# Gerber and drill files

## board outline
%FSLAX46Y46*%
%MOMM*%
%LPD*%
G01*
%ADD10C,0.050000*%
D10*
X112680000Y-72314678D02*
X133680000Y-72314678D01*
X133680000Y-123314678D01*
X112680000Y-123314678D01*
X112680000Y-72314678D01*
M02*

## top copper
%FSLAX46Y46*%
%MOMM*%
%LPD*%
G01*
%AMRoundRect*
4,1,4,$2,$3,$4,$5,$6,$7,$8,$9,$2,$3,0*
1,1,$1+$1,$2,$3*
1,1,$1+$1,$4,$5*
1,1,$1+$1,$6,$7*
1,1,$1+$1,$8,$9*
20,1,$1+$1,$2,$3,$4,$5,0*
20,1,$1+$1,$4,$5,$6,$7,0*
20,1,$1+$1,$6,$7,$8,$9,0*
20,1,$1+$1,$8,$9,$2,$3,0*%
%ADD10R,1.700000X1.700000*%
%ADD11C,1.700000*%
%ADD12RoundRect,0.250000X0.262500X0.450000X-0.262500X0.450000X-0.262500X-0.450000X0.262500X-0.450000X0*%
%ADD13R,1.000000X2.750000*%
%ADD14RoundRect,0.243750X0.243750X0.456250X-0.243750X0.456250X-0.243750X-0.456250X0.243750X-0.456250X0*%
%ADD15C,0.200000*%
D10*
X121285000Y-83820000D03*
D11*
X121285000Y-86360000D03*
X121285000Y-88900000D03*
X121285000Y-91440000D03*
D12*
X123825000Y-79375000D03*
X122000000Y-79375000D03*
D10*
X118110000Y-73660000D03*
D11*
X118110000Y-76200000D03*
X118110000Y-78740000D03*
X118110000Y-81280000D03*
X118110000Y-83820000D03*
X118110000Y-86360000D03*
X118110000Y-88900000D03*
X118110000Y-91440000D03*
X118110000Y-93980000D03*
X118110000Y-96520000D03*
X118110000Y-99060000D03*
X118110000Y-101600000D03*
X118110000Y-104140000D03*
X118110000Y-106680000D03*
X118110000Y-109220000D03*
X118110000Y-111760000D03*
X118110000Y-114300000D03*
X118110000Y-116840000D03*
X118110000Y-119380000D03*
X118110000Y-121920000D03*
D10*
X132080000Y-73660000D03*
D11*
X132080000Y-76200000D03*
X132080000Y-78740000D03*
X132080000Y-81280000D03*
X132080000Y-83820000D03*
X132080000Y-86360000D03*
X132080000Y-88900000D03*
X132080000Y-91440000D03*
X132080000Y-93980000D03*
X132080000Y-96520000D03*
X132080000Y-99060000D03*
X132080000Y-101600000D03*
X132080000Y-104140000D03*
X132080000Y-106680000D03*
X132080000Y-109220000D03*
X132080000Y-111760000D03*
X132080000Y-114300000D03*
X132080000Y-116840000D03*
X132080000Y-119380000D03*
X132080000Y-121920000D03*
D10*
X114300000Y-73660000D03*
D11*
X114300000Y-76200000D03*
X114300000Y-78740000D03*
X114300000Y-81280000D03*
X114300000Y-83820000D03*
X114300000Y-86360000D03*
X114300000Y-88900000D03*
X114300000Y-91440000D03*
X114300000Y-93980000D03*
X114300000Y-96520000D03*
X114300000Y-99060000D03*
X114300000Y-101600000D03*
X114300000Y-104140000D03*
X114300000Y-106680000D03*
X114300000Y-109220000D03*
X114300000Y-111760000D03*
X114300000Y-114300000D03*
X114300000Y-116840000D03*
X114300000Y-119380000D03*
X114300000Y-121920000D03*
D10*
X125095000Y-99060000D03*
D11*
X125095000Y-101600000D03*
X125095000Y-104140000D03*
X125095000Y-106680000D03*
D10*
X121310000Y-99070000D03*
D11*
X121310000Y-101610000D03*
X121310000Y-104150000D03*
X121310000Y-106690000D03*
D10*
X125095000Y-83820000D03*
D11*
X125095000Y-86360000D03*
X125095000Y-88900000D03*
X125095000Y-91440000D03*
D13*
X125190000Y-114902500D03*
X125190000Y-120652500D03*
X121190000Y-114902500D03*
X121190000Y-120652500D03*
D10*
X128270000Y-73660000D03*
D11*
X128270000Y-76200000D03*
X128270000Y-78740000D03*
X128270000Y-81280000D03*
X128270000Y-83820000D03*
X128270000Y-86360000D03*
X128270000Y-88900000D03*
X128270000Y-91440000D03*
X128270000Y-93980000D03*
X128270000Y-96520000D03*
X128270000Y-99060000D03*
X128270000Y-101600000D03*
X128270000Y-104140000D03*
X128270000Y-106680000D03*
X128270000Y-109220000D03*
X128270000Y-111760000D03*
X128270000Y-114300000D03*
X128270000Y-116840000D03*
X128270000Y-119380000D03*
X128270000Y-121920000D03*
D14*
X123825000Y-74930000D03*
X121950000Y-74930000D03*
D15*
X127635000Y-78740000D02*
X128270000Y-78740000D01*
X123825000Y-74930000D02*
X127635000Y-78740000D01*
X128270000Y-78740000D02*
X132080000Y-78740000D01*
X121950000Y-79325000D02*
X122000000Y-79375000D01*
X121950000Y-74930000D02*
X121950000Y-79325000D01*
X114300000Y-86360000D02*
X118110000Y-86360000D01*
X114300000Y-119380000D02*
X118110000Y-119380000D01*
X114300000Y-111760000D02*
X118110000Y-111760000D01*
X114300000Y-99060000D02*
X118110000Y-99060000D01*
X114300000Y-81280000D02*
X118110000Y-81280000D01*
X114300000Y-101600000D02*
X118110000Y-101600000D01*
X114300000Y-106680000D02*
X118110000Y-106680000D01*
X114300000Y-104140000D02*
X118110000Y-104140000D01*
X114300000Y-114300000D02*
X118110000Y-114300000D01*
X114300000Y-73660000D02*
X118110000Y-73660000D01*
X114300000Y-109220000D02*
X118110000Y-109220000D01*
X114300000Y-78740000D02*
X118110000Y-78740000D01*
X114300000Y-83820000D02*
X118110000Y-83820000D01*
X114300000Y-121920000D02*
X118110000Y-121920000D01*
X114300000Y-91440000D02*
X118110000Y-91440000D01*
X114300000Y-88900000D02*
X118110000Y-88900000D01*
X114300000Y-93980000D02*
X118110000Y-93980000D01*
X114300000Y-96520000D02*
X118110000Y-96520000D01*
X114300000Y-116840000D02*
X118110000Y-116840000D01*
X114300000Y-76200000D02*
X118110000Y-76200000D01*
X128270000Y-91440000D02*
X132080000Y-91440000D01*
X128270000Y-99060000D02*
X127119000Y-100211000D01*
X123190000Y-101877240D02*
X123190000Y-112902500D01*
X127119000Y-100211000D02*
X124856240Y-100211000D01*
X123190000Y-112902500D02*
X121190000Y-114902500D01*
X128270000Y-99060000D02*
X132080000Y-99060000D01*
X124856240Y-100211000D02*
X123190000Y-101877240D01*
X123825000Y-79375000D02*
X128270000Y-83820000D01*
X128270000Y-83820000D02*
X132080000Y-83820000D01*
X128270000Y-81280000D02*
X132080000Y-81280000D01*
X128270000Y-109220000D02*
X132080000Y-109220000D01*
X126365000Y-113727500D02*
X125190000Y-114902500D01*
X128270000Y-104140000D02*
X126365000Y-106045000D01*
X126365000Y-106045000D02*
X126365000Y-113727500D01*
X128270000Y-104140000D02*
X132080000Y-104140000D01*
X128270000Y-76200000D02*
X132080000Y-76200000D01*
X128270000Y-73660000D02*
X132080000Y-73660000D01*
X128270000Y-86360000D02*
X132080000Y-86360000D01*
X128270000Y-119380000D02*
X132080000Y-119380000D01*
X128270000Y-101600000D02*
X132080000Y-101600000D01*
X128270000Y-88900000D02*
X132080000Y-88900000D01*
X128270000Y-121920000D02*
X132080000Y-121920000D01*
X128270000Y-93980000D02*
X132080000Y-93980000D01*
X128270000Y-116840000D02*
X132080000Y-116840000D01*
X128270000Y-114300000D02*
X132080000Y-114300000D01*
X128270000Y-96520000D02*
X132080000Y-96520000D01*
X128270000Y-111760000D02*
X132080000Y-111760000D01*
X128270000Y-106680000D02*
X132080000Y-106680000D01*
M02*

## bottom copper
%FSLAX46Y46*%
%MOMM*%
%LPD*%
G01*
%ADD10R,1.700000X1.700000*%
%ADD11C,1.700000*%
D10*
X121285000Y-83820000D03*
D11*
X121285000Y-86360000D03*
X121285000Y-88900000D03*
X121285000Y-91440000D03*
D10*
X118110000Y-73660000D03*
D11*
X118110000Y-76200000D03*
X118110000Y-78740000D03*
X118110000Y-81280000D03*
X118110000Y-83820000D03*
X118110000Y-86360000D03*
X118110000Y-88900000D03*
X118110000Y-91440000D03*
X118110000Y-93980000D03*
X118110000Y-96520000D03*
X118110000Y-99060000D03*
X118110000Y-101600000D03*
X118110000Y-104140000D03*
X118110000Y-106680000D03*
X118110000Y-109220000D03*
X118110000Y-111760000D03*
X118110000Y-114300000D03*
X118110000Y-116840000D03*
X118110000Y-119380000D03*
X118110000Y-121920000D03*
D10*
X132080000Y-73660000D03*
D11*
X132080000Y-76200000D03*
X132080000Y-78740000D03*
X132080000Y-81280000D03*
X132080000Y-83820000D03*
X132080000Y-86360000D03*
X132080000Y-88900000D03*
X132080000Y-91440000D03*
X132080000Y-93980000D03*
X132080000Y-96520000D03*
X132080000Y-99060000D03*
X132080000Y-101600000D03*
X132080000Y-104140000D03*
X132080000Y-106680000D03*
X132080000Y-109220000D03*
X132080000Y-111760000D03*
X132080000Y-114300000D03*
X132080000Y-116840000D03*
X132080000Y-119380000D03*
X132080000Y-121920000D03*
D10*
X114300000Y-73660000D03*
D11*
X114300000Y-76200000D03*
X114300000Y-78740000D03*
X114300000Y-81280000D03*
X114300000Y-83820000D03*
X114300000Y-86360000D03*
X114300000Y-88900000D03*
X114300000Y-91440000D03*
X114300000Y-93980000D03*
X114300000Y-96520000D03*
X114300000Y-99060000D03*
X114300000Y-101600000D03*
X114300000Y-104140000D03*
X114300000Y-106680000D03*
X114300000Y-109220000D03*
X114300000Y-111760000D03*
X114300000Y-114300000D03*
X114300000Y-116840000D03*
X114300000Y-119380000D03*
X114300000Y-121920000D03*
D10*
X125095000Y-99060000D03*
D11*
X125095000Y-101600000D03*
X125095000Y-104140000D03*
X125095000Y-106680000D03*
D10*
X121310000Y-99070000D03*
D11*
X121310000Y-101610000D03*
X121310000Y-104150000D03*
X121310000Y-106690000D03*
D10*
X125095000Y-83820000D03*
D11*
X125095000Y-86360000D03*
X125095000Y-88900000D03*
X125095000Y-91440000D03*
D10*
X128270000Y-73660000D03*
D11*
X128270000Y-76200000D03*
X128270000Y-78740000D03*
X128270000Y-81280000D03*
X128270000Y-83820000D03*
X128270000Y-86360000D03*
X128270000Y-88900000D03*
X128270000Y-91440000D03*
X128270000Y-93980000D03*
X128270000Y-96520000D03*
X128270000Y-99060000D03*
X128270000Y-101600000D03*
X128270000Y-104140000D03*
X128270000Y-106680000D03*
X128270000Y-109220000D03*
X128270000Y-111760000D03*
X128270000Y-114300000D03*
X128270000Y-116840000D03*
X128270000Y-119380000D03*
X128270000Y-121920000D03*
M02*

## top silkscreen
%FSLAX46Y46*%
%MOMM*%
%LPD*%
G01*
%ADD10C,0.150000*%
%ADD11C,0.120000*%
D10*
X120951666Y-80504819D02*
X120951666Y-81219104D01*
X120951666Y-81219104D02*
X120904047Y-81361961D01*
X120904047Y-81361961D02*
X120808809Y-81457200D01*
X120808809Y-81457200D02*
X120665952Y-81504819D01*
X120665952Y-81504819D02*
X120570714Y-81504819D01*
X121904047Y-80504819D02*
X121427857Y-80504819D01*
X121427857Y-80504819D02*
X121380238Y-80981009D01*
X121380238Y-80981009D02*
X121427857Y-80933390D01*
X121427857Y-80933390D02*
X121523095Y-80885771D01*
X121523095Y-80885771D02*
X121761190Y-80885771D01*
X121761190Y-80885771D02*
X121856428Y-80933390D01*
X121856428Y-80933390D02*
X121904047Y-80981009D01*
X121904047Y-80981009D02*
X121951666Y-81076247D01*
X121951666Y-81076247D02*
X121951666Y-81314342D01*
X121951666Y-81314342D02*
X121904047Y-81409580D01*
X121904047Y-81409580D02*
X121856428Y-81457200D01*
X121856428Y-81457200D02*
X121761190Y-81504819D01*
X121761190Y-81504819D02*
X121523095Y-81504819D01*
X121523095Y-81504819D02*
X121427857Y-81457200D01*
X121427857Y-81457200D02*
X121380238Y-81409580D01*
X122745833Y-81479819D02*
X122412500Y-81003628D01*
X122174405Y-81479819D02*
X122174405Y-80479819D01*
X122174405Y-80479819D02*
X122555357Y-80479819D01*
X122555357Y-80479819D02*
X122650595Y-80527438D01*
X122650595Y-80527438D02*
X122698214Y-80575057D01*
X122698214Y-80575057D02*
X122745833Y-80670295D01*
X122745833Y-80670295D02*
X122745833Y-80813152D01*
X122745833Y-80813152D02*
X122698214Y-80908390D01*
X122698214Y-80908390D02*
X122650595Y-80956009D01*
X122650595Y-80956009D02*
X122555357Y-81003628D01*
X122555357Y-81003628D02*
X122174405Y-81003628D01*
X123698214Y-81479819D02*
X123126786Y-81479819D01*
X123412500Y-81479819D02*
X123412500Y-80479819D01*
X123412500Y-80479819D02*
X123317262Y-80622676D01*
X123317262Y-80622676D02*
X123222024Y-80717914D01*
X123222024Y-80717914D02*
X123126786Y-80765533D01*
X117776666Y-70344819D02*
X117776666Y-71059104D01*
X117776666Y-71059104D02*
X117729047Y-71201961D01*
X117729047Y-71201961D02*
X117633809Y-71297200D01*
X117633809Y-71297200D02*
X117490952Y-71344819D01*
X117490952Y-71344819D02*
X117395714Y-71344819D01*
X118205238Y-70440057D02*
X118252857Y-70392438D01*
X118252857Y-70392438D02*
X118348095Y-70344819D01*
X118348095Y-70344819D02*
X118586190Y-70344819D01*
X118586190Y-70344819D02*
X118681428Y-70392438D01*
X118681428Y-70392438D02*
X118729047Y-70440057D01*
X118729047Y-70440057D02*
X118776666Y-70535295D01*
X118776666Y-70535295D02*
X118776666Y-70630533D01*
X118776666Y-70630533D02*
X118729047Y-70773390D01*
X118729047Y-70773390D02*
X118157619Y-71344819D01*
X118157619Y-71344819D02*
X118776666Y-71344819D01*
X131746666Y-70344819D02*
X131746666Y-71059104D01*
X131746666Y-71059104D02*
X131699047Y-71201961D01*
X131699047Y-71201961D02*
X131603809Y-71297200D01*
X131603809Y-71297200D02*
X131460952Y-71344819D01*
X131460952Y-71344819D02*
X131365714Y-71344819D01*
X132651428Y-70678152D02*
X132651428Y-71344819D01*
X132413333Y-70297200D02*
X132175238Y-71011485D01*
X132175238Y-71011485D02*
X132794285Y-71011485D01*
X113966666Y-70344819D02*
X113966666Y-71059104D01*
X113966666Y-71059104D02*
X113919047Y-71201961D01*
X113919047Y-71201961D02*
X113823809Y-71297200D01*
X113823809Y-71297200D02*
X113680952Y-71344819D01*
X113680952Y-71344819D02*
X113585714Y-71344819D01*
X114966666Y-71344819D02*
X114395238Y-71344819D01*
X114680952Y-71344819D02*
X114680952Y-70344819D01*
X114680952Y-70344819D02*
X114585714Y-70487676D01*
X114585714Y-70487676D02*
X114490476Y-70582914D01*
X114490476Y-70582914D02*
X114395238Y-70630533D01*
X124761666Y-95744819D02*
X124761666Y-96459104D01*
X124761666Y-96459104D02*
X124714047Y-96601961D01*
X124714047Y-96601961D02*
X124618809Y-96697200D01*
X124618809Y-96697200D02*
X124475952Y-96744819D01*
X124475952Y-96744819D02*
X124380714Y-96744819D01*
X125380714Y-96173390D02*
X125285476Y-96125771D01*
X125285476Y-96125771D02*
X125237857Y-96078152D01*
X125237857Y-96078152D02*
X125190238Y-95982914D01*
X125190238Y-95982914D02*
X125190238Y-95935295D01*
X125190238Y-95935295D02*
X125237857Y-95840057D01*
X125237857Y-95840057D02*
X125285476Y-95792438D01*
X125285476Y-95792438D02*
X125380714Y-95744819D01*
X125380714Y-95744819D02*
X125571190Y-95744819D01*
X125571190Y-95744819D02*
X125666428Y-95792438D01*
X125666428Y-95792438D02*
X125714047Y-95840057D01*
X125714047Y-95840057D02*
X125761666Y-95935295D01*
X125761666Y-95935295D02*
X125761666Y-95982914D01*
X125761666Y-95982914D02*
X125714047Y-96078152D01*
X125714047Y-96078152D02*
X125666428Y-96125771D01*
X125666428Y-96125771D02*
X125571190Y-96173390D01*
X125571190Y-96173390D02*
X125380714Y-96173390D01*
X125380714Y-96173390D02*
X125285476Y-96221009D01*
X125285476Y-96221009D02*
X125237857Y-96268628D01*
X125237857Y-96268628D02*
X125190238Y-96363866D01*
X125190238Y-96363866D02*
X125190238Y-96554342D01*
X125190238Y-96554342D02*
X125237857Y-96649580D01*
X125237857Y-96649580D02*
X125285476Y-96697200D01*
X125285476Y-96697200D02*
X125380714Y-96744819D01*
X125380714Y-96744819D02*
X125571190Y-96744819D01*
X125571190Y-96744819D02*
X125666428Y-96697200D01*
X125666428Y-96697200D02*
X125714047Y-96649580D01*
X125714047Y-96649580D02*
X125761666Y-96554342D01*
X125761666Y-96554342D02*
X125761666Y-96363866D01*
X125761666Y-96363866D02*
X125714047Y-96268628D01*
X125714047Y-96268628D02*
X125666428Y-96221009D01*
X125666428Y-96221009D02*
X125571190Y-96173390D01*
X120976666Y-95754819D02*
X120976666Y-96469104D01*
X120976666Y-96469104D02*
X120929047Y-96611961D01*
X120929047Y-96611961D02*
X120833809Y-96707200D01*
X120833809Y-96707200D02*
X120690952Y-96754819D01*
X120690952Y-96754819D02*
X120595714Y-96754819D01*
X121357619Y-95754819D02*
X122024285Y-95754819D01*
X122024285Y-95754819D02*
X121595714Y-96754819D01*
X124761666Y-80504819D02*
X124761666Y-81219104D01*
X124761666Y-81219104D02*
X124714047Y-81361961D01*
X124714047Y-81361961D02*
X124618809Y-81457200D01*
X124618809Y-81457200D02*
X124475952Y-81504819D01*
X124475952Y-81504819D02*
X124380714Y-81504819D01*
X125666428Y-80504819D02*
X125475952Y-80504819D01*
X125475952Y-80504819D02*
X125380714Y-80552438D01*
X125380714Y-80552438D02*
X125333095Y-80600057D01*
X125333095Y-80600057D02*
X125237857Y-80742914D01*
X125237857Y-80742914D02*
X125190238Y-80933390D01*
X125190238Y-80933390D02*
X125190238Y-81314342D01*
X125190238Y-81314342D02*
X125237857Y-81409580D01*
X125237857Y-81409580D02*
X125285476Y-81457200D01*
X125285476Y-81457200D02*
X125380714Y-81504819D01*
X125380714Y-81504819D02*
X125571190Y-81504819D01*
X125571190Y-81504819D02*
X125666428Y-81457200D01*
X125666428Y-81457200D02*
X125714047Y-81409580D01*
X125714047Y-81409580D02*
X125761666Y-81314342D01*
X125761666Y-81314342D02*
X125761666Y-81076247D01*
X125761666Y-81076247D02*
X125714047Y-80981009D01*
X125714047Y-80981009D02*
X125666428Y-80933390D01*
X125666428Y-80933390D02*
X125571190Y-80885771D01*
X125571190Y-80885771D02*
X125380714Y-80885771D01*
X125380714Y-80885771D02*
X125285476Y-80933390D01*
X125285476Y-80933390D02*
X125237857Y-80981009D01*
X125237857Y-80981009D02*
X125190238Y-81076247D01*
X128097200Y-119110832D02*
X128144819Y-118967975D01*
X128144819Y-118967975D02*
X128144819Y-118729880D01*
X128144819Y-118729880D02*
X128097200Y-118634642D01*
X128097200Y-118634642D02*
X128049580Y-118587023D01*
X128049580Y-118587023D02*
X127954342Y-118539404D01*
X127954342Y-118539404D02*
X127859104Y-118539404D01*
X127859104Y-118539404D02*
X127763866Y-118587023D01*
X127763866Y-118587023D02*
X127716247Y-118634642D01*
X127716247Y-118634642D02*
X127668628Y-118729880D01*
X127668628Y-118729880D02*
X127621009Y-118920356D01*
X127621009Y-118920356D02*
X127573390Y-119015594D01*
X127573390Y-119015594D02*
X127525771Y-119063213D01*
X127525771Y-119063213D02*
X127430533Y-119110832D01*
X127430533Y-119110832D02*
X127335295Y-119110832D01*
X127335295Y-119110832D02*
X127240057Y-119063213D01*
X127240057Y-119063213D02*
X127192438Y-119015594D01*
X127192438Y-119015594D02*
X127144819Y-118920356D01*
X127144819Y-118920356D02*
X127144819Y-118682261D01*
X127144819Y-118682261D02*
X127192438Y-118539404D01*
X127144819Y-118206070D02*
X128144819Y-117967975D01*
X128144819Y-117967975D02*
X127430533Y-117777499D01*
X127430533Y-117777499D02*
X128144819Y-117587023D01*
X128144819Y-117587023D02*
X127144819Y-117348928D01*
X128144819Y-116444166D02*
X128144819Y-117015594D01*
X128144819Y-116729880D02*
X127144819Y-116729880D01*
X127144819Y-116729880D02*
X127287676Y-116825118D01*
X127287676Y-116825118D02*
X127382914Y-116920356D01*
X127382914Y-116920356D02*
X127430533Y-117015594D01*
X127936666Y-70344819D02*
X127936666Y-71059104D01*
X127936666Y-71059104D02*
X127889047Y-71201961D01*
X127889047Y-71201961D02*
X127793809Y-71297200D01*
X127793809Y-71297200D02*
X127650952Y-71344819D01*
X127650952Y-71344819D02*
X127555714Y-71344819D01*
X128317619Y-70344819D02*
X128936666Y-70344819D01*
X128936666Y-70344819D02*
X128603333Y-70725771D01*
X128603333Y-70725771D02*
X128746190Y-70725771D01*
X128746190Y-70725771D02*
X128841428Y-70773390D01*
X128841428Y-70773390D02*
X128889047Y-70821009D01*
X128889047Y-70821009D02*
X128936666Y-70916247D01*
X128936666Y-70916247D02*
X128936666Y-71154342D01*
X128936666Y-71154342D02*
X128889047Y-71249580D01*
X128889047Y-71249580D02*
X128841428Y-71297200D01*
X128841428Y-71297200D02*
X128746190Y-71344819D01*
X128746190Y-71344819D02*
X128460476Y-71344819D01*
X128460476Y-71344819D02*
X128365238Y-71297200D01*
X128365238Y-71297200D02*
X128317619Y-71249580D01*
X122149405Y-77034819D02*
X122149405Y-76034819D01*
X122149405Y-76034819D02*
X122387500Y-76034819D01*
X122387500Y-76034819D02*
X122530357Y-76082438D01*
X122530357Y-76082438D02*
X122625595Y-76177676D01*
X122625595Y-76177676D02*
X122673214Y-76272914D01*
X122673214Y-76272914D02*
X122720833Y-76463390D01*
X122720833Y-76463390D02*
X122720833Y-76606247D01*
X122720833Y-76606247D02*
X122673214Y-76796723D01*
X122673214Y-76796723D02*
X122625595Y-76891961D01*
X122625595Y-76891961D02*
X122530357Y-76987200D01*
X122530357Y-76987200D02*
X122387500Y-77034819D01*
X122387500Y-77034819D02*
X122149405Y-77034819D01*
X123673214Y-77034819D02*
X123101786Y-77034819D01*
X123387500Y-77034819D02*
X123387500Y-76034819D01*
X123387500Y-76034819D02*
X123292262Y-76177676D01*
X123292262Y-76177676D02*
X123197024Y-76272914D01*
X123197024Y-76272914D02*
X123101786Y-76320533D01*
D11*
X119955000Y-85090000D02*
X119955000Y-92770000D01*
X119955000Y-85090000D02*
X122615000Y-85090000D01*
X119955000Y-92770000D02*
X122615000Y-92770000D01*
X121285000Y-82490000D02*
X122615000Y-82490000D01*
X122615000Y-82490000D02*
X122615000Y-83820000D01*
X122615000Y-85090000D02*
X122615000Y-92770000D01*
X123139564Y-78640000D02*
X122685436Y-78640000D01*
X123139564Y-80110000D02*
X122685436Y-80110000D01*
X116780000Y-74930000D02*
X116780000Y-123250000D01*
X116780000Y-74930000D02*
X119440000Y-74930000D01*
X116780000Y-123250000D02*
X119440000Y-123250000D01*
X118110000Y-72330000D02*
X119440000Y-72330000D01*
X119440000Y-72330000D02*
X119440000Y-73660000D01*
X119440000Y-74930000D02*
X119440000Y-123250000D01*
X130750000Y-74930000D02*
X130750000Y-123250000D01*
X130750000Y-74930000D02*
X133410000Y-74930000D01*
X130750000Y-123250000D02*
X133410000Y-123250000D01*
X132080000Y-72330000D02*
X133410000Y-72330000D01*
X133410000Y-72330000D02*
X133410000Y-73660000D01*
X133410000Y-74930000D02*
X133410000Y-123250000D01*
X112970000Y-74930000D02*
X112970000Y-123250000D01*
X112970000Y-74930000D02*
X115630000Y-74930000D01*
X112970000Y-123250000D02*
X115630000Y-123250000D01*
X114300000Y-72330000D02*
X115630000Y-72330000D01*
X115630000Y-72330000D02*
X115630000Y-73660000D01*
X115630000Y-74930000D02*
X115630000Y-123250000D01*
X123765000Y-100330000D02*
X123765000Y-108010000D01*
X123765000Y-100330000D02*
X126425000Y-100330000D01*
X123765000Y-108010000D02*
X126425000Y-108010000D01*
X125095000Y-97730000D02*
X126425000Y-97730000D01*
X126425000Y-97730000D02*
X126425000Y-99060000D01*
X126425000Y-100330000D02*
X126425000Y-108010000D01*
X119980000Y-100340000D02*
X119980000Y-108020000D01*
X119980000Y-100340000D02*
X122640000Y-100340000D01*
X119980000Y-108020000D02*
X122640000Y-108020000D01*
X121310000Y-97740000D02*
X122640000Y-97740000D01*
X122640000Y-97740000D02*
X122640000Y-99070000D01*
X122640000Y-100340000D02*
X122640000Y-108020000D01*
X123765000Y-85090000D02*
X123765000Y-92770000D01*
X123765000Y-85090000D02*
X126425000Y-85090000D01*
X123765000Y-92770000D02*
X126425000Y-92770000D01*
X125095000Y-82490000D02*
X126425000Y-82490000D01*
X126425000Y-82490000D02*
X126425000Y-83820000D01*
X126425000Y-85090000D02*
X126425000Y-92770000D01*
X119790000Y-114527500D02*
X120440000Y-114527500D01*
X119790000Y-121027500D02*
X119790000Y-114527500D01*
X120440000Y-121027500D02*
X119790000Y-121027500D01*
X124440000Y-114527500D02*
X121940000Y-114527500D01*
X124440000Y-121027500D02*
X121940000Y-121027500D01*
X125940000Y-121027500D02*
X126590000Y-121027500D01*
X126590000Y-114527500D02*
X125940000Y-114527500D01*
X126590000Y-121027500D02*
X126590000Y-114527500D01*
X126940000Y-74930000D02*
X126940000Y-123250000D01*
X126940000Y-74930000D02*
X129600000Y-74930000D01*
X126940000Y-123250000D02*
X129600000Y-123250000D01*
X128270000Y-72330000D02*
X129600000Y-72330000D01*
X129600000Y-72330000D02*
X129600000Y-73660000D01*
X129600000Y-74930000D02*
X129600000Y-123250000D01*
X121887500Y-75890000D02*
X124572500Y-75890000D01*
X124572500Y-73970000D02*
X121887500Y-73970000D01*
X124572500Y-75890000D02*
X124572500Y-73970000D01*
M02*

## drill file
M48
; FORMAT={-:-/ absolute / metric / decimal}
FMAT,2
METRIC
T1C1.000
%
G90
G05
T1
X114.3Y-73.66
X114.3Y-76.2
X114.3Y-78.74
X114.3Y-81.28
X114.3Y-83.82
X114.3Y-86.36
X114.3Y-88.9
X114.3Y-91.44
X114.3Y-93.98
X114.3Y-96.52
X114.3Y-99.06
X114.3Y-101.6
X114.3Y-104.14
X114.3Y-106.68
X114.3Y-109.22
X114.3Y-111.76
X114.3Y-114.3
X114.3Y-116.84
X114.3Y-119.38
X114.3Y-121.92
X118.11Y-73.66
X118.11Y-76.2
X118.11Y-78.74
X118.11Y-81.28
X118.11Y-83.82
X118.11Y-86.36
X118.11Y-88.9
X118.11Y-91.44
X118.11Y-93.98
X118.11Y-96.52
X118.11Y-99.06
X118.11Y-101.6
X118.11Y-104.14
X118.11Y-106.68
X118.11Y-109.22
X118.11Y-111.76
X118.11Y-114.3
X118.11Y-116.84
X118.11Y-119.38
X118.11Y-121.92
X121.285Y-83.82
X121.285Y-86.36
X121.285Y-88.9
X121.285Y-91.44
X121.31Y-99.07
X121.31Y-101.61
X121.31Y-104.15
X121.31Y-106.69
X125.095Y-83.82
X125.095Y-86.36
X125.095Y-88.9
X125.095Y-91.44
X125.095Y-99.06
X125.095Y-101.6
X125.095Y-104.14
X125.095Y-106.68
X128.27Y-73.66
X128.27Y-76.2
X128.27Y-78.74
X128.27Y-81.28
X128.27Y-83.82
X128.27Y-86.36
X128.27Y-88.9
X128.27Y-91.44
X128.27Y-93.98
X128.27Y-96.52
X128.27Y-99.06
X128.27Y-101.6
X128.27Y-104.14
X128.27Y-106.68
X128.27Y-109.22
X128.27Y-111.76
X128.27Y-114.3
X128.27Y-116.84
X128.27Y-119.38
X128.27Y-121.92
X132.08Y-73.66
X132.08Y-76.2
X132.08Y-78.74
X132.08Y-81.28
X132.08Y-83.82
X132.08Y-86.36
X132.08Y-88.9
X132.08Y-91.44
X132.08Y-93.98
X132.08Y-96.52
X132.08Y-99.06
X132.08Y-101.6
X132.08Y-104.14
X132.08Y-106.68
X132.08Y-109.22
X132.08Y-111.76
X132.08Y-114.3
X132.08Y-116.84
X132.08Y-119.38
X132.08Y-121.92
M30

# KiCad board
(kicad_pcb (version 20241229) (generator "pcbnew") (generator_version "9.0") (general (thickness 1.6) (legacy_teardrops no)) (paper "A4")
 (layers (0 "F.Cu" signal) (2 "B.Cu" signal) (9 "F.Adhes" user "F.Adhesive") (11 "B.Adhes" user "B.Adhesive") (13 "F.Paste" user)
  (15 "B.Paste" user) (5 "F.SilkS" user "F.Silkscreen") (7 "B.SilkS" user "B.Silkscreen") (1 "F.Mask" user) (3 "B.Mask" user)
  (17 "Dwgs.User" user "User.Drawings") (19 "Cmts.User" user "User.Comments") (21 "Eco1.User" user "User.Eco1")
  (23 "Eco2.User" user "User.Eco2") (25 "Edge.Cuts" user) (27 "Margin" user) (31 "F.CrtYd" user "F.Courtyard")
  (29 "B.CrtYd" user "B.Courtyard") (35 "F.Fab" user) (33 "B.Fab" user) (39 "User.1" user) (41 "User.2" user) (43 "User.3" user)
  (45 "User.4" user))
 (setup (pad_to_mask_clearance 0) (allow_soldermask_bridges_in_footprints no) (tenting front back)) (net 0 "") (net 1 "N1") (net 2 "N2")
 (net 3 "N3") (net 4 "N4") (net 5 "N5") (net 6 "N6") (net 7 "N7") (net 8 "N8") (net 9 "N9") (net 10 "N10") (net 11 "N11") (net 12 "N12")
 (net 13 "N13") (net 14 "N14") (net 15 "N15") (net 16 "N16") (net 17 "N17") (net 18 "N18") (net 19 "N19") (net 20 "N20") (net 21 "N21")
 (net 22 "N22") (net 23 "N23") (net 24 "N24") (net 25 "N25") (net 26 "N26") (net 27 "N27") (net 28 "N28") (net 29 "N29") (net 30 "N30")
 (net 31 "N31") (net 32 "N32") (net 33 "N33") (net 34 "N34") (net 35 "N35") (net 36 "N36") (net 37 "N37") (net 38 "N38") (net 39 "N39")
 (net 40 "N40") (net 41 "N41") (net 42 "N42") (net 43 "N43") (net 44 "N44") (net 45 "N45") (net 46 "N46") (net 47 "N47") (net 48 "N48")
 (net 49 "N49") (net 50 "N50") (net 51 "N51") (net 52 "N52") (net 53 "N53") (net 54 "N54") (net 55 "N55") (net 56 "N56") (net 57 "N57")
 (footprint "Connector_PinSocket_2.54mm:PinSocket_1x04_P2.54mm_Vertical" (layer "F.Cu") (at 121.285 83.82)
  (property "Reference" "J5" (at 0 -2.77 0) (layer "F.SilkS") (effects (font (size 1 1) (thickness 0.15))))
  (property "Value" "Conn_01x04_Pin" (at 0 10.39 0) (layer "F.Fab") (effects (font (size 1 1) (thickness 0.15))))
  (fp_line (start -1.33 1.27) (end -1.33 8.95) (stroke (width 0.12) (type solid)) (layer "F.SilkS"))
  (fp_line (start -1.33 1.27) (end 1.33 1.27) (stroke (width 0.12) (type solid)) (layer "F.SilkS"))
  (fp_line (start -1.33 8.95) (end 1.33 8.95) (stroke (width 0.12) (type solid)) (layer "F.SilkS"))
  (fp_line (start 0 -1.33) (end 1.33 -1.33) (stroke (width 0.12) (type solid)) (layer "F.SilkS"))
  (fp_line (start 1.33 -1.33) (end 1.33 0) (stroke (width 0.12) (type solid)) (layer "F.SilkS"))
  (fp_line (start 1.33 1.27) (end 1.33 8.95) (stroke (width 0.12) (type solid)) (layer "F.SilkS"))
  (pad "1" thru_hole rect (at 0 0) (size 1.7 1.7) (drill 1) (layers "*.Cu" "*.Mask") (remove_unused_layers no) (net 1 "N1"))
  (pad "2" thru_hole circle (at 0 2.54) (size 1.7 1.7) (drill 1) (layers "*.Cu" "*.Mask") (remove_unused_layers no) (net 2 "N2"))
  (pad "3" thru_hole circle (at 0 5.08) (size 1.7 1.7) (drill 1) (layers "*.Cu" "*.Mask") (remove_unused_layers no) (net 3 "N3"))
  (pad "4" thru_hole circle (at 0 7.62) (size 1.7 1.7) (drill 1) (layers "*.Cu" "*.Mask") (remove_unused_layers no) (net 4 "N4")))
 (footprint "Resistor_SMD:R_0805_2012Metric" (layer "F.Cu") (at 122.9125 79.375 180)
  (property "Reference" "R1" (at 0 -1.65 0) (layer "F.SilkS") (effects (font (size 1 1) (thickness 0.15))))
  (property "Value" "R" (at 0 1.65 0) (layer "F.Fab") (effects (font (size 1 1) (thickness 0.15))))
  (fp_line (start -0.227064 0.735) (end 0.227064 0.735) (stroke (width 0.12) (type solid)) (layer "F.SilkS"))
  (fp_line (start -0.227064 -0.735) (end 0.227064 -0.735) (stroke (width 0.12) (type solid)) (layer "F.SilkS"))
  (pad "1" smd roundrect (at -0.9125 0 180) (size 1.025 1.4) (layers "F.Cu" "F.Mask" "F.Paste") (roundrect_rratio 0.243902) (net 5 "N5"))
  (pad "2" smd roundrect (at 0.9125 0 180) (size 1.025 1.4) (layers "F.Cu" "F.Mask" "F.Paste") (roundrect_rratio 0.243902) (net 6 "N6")))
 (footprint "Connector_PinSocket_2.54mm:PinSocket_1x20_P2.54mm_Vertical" (layer "F.Cu") (at 118.11 73.66)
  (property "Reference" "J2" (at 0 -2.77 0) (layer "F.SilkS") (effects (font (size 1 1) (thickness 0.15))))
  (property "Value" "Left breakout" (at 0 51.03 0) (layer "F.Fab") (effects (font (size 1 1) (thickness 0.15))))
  (fp_line (start -1.33 1.27) (end -1.33 49.59) (stroke (width 0.12) (type solid)) (layer "F.SilkS"))
  (fp_line (start -1.33 1.27) (end 1.33 1.27) (stroke (width 0.12) (type solid)) (layer "F.SilkS"))
  (fp_line (start -1.33 49.59) (end 1.33 49.59) (stroke (width 0.12) (type solid)) (layer "F.SilkS"))
  (fp_line (start 0 -1.33) (end 1.33 -1.33) (stroke (width 0.12) (type solid)) (layer "F.SilkS"))
  (fp_line (start 1.33 -1.33) (end 1.33 0) (stroke (width 0.12) (type solid)) (layer "F.SilkS"))
  (fp_line (start 1.33 1.27) (end 1.33 49.59) (stroke (width 0.12) (type solid)) (layer "F.SilkS"))
  (pad "1" thru_hole rect (at 0 0) (size 1.7 1.7) (drill 1) (layers "*.Cu" "*.Mask") (remove_unused_layers no) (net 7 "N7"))
  (pad "2" thru_hole circle (at 0 2.54) (size 1.7 1.7) (drill 1) (layers "*.Cu" "*.Mask") (remove_unused_layers no) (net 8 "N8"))
  (pad "3" thru_hole circle (at 0 5.08) (size 1.7 1.7) (drill 1) (layers "*.Cu" "*.Mask") (remove_unused_layers no) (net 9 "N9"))
  (pad "4" thru_hole circle (at 0 7.62) (size 1.7 1.7) (drill 1) (layers "*.Cu" "*.Mask") (remove_unused_layers no) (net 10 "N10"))
  (pad "5" thru_hole circle (at 0 10.16) (size 1.7 1.7) (drill 1) (layers "*.Cu" "*.Mask") (remove_unused_layers no) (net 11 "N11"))
  (pad "6" thru_hole circle (at 0 12.7) (size 1.7 1.7) (drill 1) (layers "*.Cu" "*.Mask") (remove_unused_layers no) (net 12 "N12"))
  (pad "7" thru_hole circle (at 0 15.24) (size 1.7 1.7) (drill 1) (layers "*.Cu" "*.Mask") (remove_unused_layers no) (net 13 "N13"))
  (pad "8" thru_hole circle (at 0 17.78) (size 1.7 1.7) (drill 1) (layers "*.Cu" "*.Mask") (remove_unused_layers no) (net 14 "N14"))
  (pad "9" thru_hole circle (at 0 20.32) (size 1.7 1.7) (drill 1) (layers "*.Cu" "*.Mask") (remove_unused_layers no) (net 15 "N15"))
  (pad "10" thru_hole circle (at 0 22.86) (size 1.7 1.7) (drill 1) (layers "*.Cu" "*.Mask") (remove_unused_layers no) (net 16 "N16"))
  (pad "11" thru_hole circle (at 0 25.4) (size 1.7 1.7) (drill 1) (layers "*.Cu" "*.Mask") (remove_unused_layers no) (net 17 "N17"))
  (pad "12" thru_hole circle (at 0 27.94) (size 1.7 1.7) (drill 1) (layers "*.Cu" "*.Mask") (remove_unused_layers no) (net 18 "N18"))
  (pad "13" thru_hole circle (at 0 30.48) (size 1.7 1.7) (drill 1) (layers "*.Cu" "*.Mask") (remove_unused_layers no) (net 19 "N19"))
  (pad "14" thru_hole circle (at 0 33.02) (size 1.7 1.7) (drill 1) (layers "*.Cu" "*.Mask") (remove_unused_layers no) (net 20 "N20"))
  (pad "15" thru_hole circle (at 0 35.56) (size 1.7 1.7) (drill 1) (layers "*.Cu" "*.Mask") (remove_unused_layers no) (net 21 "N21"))
  (pad "16" thru_hole circle (at 0 38.1) (size 1.7 1.7) (drill 1) (layers "*.Cu" "*.Mask") (remove_unused_layers no) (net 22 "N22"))
  (pad "17" thru_hole circle (at 0 40.64) (size 1.7 1.7) (drill 1) (layers "*.Cu" "*.Mask") (remove_unused_layers no) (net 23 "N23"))
  (pad "18" thru_hole circle (at 0 43.18) (size 1.7 1.7) (drill 1) (layers "*.Cu" "*.Mask") (remove_unused_layers no) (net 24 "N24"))
  (pad "19" thru_hole circle (at 0 45.72) (size 1.7 1.7) (drill 1) (layers "*.Cu" "*.Mask") (remove_unused_layers no) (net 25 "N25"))
  (pad "20" thru_hole circle (at 0 48.26) (size 1.7 1.7) (drill 1) (layers "*.Cu" "*.Mask") (remove_unused_layers no) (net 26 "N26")))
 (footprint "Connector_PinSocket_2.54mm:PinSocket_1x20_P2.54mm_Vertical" (layer "F.Cu") (at 132.08 73.66)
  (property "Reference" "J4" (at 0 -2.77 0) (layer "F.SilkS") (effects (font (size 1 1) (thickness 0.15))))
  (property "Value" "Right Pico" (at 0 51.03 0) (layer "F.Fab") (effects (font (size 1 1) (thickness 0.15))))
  (fp_line (start -1.33 1.27) (end -1.33 49.59) (stroke (width 0.12) (type solid)) (layer "F.SilkS"))
  (fp_line (start -1.33 1.27) (end 1.33 1.27) (stroke (width 0.12) (type solid)) (layer "F.SilkS"))
  (fp_line (start -1.33 49.59) (end 1.33 49.59) (stroke (width 0.12) (type solid)) (layer "F.SilkS"))
  (fp_line (start 0 -1.33) (end 1.33 -1.33) (stroke (width 0.12) (type solid)) (layer "F.SilkS"))
  (fp_line (start 1.33 -1.33) (end 1.33 0) (stroke (width 0.12) (type solid)) (layer "F.SilkS"))
  (fp_line (start 1.33 1.27) (end 1.33 49.59) (stroke (width 0.12) (type solid)) (layer "F.SilkS"))
  (pad "1" thru_hole rect (at 0 0) (size 1.7 1.7) (drill 1) (layers "*.Cu" "*.Mask") (remove_unused_layers no) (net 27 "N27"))
  (pad "2" thru_hole circle (at 0 2.54) (size 1.7 1.7) (drill 1) (layers "*.Cu" "*.Mask") (remove_unused_layers no) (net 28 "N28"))
  (pad "3" thru_hole circle (at 0 5.08) (size 1.7 1.7) (drill 1) (layers "*.Cu" "*.Mask") (remove_unused_layers no) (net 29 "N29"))
  (pad "4" thru_hole circle (at 0 7.62) (size 1.7 1.7) (drill 1) (layers "*.Cu" "*.Mask") (remove_unused_layers no) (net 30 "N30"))
  (pad "5" thru_hole circle (at 0 10.16) (size 1.7 1.7) (drill 1) (layers "*.Cu" "*.Mask") (remove_unused_layers no) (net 5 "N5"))
  (pad "6" thru_hole circle (at 0 12.7) (size 1.7 1.7) (drill 1) (layers "*.Cu" "*.Mask") (remove_unused_layers no) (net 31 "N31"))
  (pad "7" thru_hole circle (at 0 15.24) (size 1.7 1.7) (drill 1) (layers "*.Cu" "*.Mask") (remove_unused_layers no) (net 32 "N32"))
  (pad "8" thru_hole circle (at 0 17.78) (size 1.7 1.7) (drill 1) (layers "*.Cu" "*.Mask") (remove_unused_layers no) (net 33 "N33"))
  (pad "9" thru_hole circle (at 0 20.32) (size 1.7 1.7) (drill 1) (layers "*.Cu" "*.Mask") (remove_unused_layers no) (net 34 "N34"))
  (pad "10" thru_hole circle (at 0 22.86) (size 1.7 1.7) (drill 1) (layers "*.Cu" "*.Mask") (remove_unused_layers no) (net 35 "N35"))
  (pad "11" thru_hole circle (at 0 25.4) (size 1.7 1.7) (drill 1) (layers "*.Cu" "*.Mask") (remove_unused_layers no) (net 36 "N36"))
  (pad "12" thru_hole circle (at 0 27.94) (size 1.7 1.7) (drill 1) (layers "*.Cu" "*.Mask") (remove_unused_layers no) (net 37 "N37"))
  (pad "13" thru_hole circle (at 0 30.48) (size 1.7 1.7) (drill 1) (layers "*.Cu" "*.Mask") (remove_unused_layers no) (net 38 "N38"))
  (pad "14" thru_hole circle (at 0 33.02) (size 1.7 1.7) (drill 1) (layers "*.Cu" "*.Mask") (remove_unused_layers no) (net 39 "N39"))
  (pad "15" thru_hole circle (at 0 35.56) (size 1.7 1.7) (drill 1) (layers "*.Cu" "*.Mask") (remove_unused_layers no) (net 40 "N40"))
  (pad "16" thru_hole circle (at 0 38.1) (size 1.7 1.7) (drill 1) (layers "*.Cu" "*.Mask") (remove_unused_layers no) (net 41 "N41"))
  (pad "17" thru_hole circle (at 0 40.64) (size 1.7 1.7) (drill 1) (layers "*.Cu" "*.Mask") (remove_unused_layers no) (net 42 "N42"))
  (pad "18" thru_hole circle (at 0 43.18) (size 1.7 1.7) (drill 1) (layers "*.Cu" "*.Mask") (remove_unused_layers no) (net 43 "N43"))
  (pad "19" thru_hole circle (at 0 45.72) (size 1.7 1.7) (drill 1) (layers "*.Cu" "*.Mask") (remove_unused_layers no) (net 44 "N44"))
  (pad "20" thru_hole circle (at 0 48.26) (size 1.7 1.7) (drill 1) (layers "*.Cu" "*.Mask") (remove_unused_layers no) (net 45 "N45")))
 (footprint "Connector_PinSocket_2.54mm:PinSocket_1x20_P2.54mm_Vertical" (layer "F.Cu") (at 114.3 73.66)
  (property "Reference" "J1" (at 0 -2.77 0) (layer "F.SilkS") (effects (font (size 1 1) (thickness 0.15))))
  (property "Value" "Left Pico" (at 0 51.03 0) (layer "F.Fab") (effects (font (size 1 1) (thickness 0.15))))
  (fp_line (start -1.33 1.27) (end -1.33 49.59) (stroke (width 0.12) (type solid)) (layer "F.SilkS"))
  (fp_line (start -1.33 1.27) (end 1.33 1.27) (stroke (width 0.12) (type solid)) (layer "F.SilkS"))
  (fp_line (start -1.33 49.59) (end 1.33 49.59) (stroke (width 0.12) (type solid)) (layer "F.SilkS"))
  (fp_line (start 0 -1.33) (end 1.33 -1.33) (stroke (width 0.12) (type solid)) (layer "F.SilkS"))
  (fp_line (start 1.33 -1.33) (end 1.33 0) (stroke (width 0.12) (type solid)) (layer "F.SilkS"))
  (fp_line (start 1.33 1.27) (end 1.33 49.59) (stroke (width 0.12) (type solid)) (layer "F.SilkS"))
  (pad "1" thru_hole rect (at 0 0) (size 1.7 1.7) (drill 1) (layers "*.Cu" "*.Mask") (remove_unused_layers no) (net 7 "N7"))
  (pad "2" thru_hole circle (at 0 2.54) (size 1.7 1.7) (drill 1) (layers "*.Cu" "*.Mask") (remove_unused_layers no) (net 8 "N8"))
  (pad "3" thru_hole circle (at 0 5.08) (size 1.7 1.7) (drill 1) (layers "*.Cu" "*.Mask") (remove_unused_layers no) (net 9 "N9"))
  (pad "4" thru_hole circle (at 0 7.62) (size 1.7 1.7) (drill 1) (layers "*.Cu" "*.Mask") (remove_unused_layers no) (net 10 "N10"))
  (pad "5" thru_hole circle (at 0 10.16) (size 1.7 1.7) (drill 1) (layers "*.Cu" "*.Mask") (remove_unused_layers no) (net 11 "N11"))
  (pad "6" thru_hole circle (at 0 12.7) (size 1.7 1.7) (drill 1) (layers "*.Cu" "*.Mask") (remove_unused_layers no) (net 12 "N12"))
  (pad "7" thru_hole circle (at 0 15.24) (size 1.7 1.7) (drill 1) (layers "*.Cu" "*.Mask") (remove_unused_layers no) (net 13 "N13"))
  (pad "8" thru_hole circle (at 0 17.78) (size 1.7 1.7) (drill 1) (layers "*.Cu" "*.Mask") (remove_unused_layers no) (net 14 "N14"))
  (pad "9" thru_hole circle (at 0 20.32) (size 1.7 1.7) (drill 1) (layers "*.Cu" "*.Mask") (remove_unused_layers no) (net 15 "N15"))
  (pad "10" thru_hole circle (at 0 22.86) (size 1.7 1.7) (drill 1) (layers "*.Cu" "*.Mask") (remove_unused_layers no) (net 16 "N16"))
  (pad "11" thru_hole circle (at 0 25.4) (size 1.7 1.7) (drill 1) (layers "*.Cu" "*.Mask") (remove_unused_layers no) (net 17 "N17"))
  (pad "12" thru_hole circle (at 0 27.94) (size 1.7 1.7) (drill 1) (layers "*.Cu" "*.Mask") (remove_unused_layers no) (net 18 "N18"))
  (pad "13" thru_hole circle (at 0 30.48) (size 1.7 1.7) (drill 1) (layers "*.Cu" "*.Mask") (remove_unused_layers no) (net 19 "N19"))
  (pad "14" thru_hole circle (at 0 33.02) (size 1.7 1.7) (drill 1) (layers "*.Cu" "*.Mask") (remove_unused_layers no) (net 20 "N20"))
  (pad "15" thru_hole circle (at 0 35.56) (size 1.7 1.7) (drill 1) (layers "*.Cu" "*.Mask") (remove_unused_layers no) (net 21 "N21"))
  (pad "16" thru_hole circle (at 0 38.1) (size 1.7 1.7) (drill 1) (layers "*.Cu" "*.Mask") (remove_unused_layers no) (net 22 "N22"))
  (pad "17" thru_hole circle (at 0 40.64) (size 1.7 1.7) (drill 1) (layers "*.Cu" "*.Mask") (remove_unused_layers no) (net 23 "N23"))
  (pad "18" thru_hole circle (at 0 43.18) (size 1.7 1.7) (drill 1) (layers "*.Cu" "*.Mask") (remove_unused_layers no) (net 24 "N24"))
  (pad "19" thru_hole circle (at 0 45.72) (size 1.7 1.7) (drill 1) (layers "*.Cu" "*.Mask") (remove_unused_layers no) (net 25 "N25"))
  (pad "20" thru_hole circle (at 0 48.26) (size 1.7 1.7) (drill 1) (layers "*.Cu" "*.Mask") (remove_unused_layers no) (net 26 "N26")))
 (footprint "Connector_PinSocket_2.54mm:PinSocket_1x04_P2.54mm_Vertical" (layer "F.Cu") (at 125.095 99.06)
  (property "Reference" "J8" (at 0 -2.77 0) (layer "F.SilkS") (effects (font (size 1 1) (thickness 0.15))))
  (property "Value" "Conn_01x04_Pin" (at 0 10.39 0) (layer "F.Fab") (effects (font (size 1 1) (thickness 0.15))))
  (fp_line (start -1.33 1.27) (end -1.33 8.95) (stroke (width 0.12) (type solid)) (layer "F.SilkS"))
  (fp_line (start -1.33 1.27) (end 1.33 1.27) (stroke (width 0.12) (type solid)) (layer "F.SilkS"))
  (fp_line (start -1.33 8.95) (end 1.33 8.95) (stroke (width 0.12) (type solid)) (layer "F.SilkS"))
  (fp_line (start 0 -1.33) (end 1.33 -1.33) (stroke (width 0.12) (type solid)) (layer "F.SilkS"))
  (fp_line (start 1.33 -1.33) (end 1.33 0) (stroke (width 0.12) (type solid)) (layer "F.SilkS"))
  (fp_line (start 1.33 1.27) (end 1.33 8.95) (stroke (width 0.12) (type solid)) (layer "F.SilkS"))
  (pad "1" thru_hole rect (at 0 0) (size 1.7 1.7) (drill 1) (layers "*.Cu" "*.Mask") (remove_unused_layers no) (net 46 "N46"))
  (pad "2" thru_hole circle (at 0 2.54) (size 1.7 1.7) (drill 1) (layers "*.Cu" "*.Mask") (remove_unused_layers no) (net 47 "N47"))
  (pad "3" thru_hole circle (at 0 5.08) (size 1.7 1.7) (drill 1) (layers "*.Cu" "*.Mask") (remove_unused_layers no) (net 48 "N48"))
  (pad "4" thru_hole circle (at 0 7.62) (size 1.7 1.7) (drill 1) (layers "*.Cu" "*.Mask") (remove_unused_layers no) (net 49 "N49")))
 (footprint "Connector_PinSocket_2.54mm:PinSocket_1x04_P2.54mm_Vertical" (layer "F.Cu") (at 121.31 99.07)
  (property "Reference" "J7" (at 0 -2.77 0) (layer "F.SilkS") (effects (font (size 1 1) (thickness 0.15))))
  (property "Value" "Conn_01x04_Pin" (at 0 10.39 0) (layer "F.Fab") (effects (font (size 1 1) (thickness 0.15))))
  (fp_line (start -1.33 1.27) (end -1.33 8.95) (stroke (width 0.12) (type solid)) (layer "F.SilkS"))
  (fp_line (start -1.33 1.27) (end 1.33 1.27) (stroke (width 0.12) (type solid)) (layer "F.SilkS"))
  (fp_line (start -1.33 8.95) (end 1.33 8.95) (stroke (width 0.12) (type solid)) (layer "F.SilkS"))
  (fp_line (start 0 -1.33) (end 1.33 -1.33) (stroke (width 0.12) (type solid)) (layer "F.SilkS"))
  (fp_line (start 1.33 -1.33) (end 1.33 0) (stroke (width 0.12) (type solid)) (layer "F.SilkS"))
  (fp_line (start 1.33 1.27) (end 1.33 8.95) (stroke (width 0.12) (type solid)) (layer "F.SilkS"))
  (pad "1" thru_hole rect (at 0 0) (size 1.7 1.7) (drill 1) (layers "*.Cu" "*.Mask") (remove_unused_layers no) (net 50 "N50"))
  (pad "2" thru_hole circle (at 0 2.54) (size 1.7 1.7) (drill 1) (layers "*.Cu" "*.Mask") (remove_unused_layers no) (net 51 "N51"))
  (pad "3" thru_hole circle (at 0 5.08) (size 1.7 1.7) (drill 1) (layers "*.Cu" "*.Mask") (remove_unused_layers no) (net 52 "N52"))
  (pad "4" thru_hole circle (at 0 7.62) (size 1.7 1.7) (drill 1) (layers "*.Cu" "*.Mask") (remove_unused_layers no) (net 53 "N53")))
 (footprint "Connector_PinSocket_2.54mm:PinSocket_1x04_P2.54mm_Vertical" (layer "F.Cu") (at 125.095 83.82)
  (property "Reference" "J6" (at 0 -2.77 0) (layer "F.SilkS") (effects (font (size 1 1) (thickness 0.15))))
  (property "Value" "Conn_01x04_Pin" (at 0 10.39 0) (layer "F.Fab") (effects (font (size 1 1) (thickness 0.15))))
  (fp_line (start -1.33 1.27) (end -1.33 8.95) (stroke (width 0.12) (type solid)) (layer "F.SilkS"))
  (fp_line (start -1.33 1.27) (end 1.33 1.27) (stroke (width 0.12) (type solid)) (layer "F.SilkS"))
  (fp_line (start -1.33 8.95) (end 1.33 8.95) (stroke (width 0.12) (type solid)) (layer "F.SilkS"))
  (fp_line (start 0 -1.33) (end 1.33 -1.33) (stroke (width 0.12) (type solid)) (layer "F.SilkS"))
  (fp_line (start 1.33 -1.33) (end 1.33 0) (stroke (width 0.12) (type solid)) (layer "F.SilkS"))
  (fp_line (start 1.33 1.27) (end 1.33 8.95) (stroke (width 0.12) (type solid)) (layer "F.SilkS"))
  (pad "1" thru_hole rect (at 0 0) (size 1.7 1.7) (drill 1) (layers "*.Cu" "*.Mask") (remove_unused_layers no) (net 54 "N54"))
  (pad "2" thru_hole circle (at 0 2.54) (size 1.7 1.7) (drill 1) (layers "*.Cu" "*.Mask") (remove_unused_layers no) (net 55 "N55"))
  (pad "3" thru_hole circle (at 0 5.08) (size 1.7 1.7) (drill 1) (layers "*.Cu" "*.Mask") (remove_unused_layers no) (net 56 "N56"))
  (pad "4" thru_hole circle (at 0 7.62) (size 1.7 1.7) (drill 1) (layers "*.Cu" "*.Mask") (remove_unused_layers no) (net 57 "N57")))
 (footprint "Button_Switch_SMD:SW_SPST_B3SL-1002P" (layer "F.Cu") (at 123.19 117.7775 -90)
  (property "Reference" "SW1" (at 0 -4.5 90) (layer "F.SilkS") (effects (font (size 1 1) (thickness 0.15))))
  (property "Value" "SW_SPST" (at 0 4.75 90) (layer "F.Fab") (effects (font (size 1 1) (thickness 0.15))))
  (fp_line (start -3.25 3.4) (end -3.25 2.75) (stroke (width 0.12) (type solid)) (layer "F.SilkS"))
  (fp_line (start 3.25 3.4) (end -3.25 3.4) (stroke (width 0.12) (type solid)) (layer "F.SilkS"))
  (fp_line (start 3.25 2.75) (end 3.25 3.4) (stroke (width 0.12) (type solid)) (layer "F.SilkS"))
  (fp_line (start -3.25 -1.25) (end -3.25 1.25) (stroke (width 0.12) (type solid)) (layer "F.SilkS"))
  (fp_line (start 3.25 -1.25) (end 3.25 1.25) (stroke (width 0.12) (type solid)) (layer "F.SilkS"))
  (fp_line (start 3.25 -2.75) (end 3.25 -3.4) (stroke (width 0.12) (type solid)) (layer "F.SilkS"))
  (fp_line (start -3.25 -3.4) (end -3.25 -2.75) (stroke (width 0.12) (type solid)) (layer "F.SilkS"))
  (fp_line (start 3.25 -3.4) (end -3.25 -3.4) (stroke (width 0.12) (type solid)) (layer "F.SilkS"))
  (pad "1" smd rect (at -2.875 -2 270) (size 2.75 1) (layers "F.Cu" "F.Mask" "F.Paste") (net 38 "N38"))
  (pad "1" smd rect (at 2.875 -2 270) (size 2.75 1) (layers "F.Cu" "F.Mask" "F.Paste") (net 38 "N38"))
  (pad "2" smd rect (at -2.875 2 270) (size 2.75 1) (layers "F.Cu" "F.Mask" "F.Paste") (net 36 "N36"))
  (pad "2" smd rect (at 2.875 2 270) (size 2.75 1) (layers "F.Cu" "F.Mask" "F.Paste") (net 36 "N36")))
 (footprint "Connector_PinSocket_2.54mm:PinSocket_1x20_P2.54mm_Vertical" (layer "F.Cu") (at 128.27 73.66)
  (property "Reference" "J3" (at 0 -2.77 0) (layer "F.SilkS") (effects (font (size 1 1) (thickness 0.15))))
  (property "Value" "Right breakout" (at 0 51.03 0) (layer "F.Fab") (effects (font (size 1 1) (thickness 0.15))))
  (fp_line (start -1.33 1.27) (end -1.33 49.59) (stroke (width 0.12) (type solid)) (layer "F.SilkS"))
  (fp_line (start -1.33 1.27) (end 1.33 1.27) (stroke (width 0.12) (type solid)) (layer "F.SilkS"))
  (fp_line (start -1.33 49.59) (end 1.33 49.59) (stroke (width 0.12) (type solid)) (layer "F.SilkS"))
  (fp_line (start 0 -1.33) (end 1.33 -1.33) (stroke (width 0.12) (type solid)) (layer "F.SilkS"))
  (fp_line (start 1.33 -1.33) (end 1.33 0) (stroke (width 0.12) (type solid)) (layer "F.SilkS"))
  (fp_line (start 1.33 1.27) (end 1.33 49.59) (stroke (width 0.12) (type solid)) (layer "F.SilkS"))
  (pad "1" thru_hole rect (at 0 0) (size 1.7 1.7) (drill 1) (layers "*.Cu" "*.Mask") (remove_unused_layers no) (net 27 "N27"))
  (pad "2" thru_hole circle (at 0 2.54) (size 1.7 1.7) (drill 1) (layers "*.Cu" "*.Mask") (remove_unused_layers no) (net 28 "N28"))
  (pad "3" thru_hole circle (at 0 5.08) (size 1.7 1.7) (drill 1) (layers "*.Cu" "*.Mask") (remove_unused_layers no) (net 29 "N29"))
  (pad "4" thru_hole circle (at 0 7.62) (size 1.7 1.7) (drill 1) (layers "*.Cu" "*.Mask") (remove_unused_layers no) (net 30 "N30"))
  (pad "5" thru_hole circle (at 0 10.16) (size 1.7 1.7) (drill 1) (layers "*.Cu" "*.Mask") (remove_unused_layers no) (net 5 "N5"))
  (pad "6" thru_hole circle (at 0 12.7) (size 1.7 1.7) (drill 1) (layers "*.Cu" "*.Mask") (remove_unused_layers no) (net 31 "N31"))
  (pad "7" thru_hole circle (at 0 15.24) (size 1.7 1.7) (drill 1) (layers "*.Cu" "*.Mask") (remove_unused_layers no) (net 32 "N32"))
  (pad "8" thru_hole circle (at 0 17.78) (size 1.7 1.7) (drill 1) (layers "*.Cu" "*.Mask") (remove_unused_layers no) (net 33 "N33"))
  (pad "9" thru_hole circle (at 0 20.32) (size 1.7 1.7) (drill 1) (layers "*.Cu" "*.Mask") (remove_unused_layers no) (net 34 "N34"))
  (pad "10" thru_hole circle (at 0 22.86) (size 1.7 1.7) (drill 1) (layers "*.Cu" "*.Mask") (remove_unused_layers no) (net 35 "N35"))
  (pad "11" thru_hole circle (at 0 25.4) (size 1.7 1.7) (drill 1) (layers "*.Cu" "*.Mask") (remove_unused_layers no) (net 36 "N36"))
  (pad "12" thru_hole circle (at 0 27.94) (size 1.7 1.7) (drill 1) (layers "*.Cu" "*.Mask") (remove_unused_layers no) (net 37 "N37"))
  (pad "13" thru_hole circle (at 0 30.48) (size 1.7 1.7) (drill 1) (layers "*.Cu" "*.Mask") (remove_unused_layers no) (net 38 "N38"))
  (pad "14" thru_hole circle (at 0 33.02) (size 1.7 1.7) (drill 1) (layers "*.Cu" "*.Mask") (remove_unused_layers no) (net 39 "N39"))
  (pad "15" thru_hole circle (at 0 35.56) (size 1.7 1.7) (drill 1) (layers "*.Cu" "*.Mask") (remove_unused_layers no) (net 40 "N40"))
  (pad "16" thru_hole circle (at 0 38.1) (size 1.7 1.7) (drill 1) (layers "*.Cu" "*.Mask") (remove_unused_layers no) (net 41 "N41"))
  (pad "17" thru_hole circle (at 0 40.64) (size 1.7 1.7) (drill 1) (layers "*.Cu" "*.Mask") (remove_unused_layers no) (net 42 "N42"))
  (pad "18" thru_hole circle (at 0 43.18) (size 1.7 1.7) (drill 1) (layers "*.Cu" "*.Mask") (remove_unused_layers no) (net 43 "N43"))
  (pad "19" thru_hole circle (at 0 45.72) (size 1.7 1.7) (drill 1) (layers "*.Cu" "*.Mask") (remove_unused_layers no) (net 44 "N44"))
  (pad "20" thru_hole circle (at 0 48.26) (size 1.7 1.7) (drill 1) (layers "*.Cu" "*.Mask") (remove_unused_layers no) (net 45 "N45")))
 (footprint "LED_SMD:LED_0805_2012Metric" (layer "F.Cu") (at 122.8875 74.93 180)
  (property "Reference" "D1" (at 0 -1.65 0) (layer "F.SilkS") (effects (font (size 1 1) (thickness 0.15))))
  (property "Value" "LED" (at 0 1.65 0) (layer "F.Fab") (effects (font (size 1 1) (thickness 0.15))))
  (fp_line (start 1 -0.96) (end -1.685 -0.96) (stroke (width 0.12) (type solid)) (layer "F.SilkS"))
  (fp_line (start -1.685 0.96) (end 1 0.96) (stroke (width 0.12) (type solid)) (layer "F.SilkS"))
  (fp_line (start -1.685 -0.96) (end -1.685 0.96) (stroke (width 0.12) (type solid)) (layer "F.SilkS"))
  (pad "1" smd roundrect (at -0.9375 0 180) (size 0.975 1.4) (layers "F.Cu" "F.Mask" "F.Paste") (roundrect_rratio 0.25) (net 29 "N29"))
  (pad "2" smd roundrect (at 0.9375 0 180) (size 0.975 1.4) (layers "F.Cu" "F.Mask" "F.Paste") (roundrect_rratio 0.25) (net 6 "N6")))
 (gr_rect (start 112.68 72.314678) (end 133.68 123.314678) (stroke (width 0.05) (type default)) (fill no) (layer "Edge.Cuts"))
 (segment (start 127.635 78.74) (end 128.27 78.74) (width 0.2) (layer "F.Cu") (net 29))
 (segment (start 123.825 74.93) (end 127.635 78.74) (width 0.2) (layer "F.Cu") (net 29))
 (segment (start 128.27 78.74) (end 132.08 78.74) (width 0.2) (layer "F.Cu") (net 29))
 (segment (start 121.95 79.325) (end 122 79.375) (width 0.2) (layer "F.Cu") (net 6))
 (segment (start 121.95 74.93) (end 121.95 79.325) (width 0.2) (layer "F.Cu") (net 6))
 (segment (start 114.3 86.36) (end 118.11 86.36) (width 0.2) (layer "F.Cu") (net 12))
 (segment (start 114.3 119.38) (end 118.11 119.38) (width 0.2) (layer "F.Cu") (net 25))
 (segment (start 114.3 111.76) (end 118.11 111.76) (width 0.2) (layer "F.Cu") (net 22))
 (segment (start 114.3 99.06) (end 118.11 99.06) (width 0.2) (layer "F.Cu") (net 17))
 (segment (start 114.3 81.28) (end 118.11 81.28) (width 0.2) (layer "F.Cu") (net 10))
 (segment (start 114.3 101.6) (end 118.11 101.6) (width 0.2) (layer "F.Cu") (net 18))
 (segment (start 114.3 106.68) (end 118.11 106.68) (width 0.2) (layer "F.Cu") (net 20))
 (segment (start 114.3 104.14) (end 118.11 104.14) (width 0.2) (layer "F.Cu") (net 19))
 (segment (start 114.3 114.3) (end 118.11 114.3) (width 0.2) (layer "F.Cu") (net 23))
 (segment (start 114.3 73.66) (end 118.11 73.66) (width 0.2) (layer "F.Cu") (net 7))
 (segment (start 114.3 109.22) (end 118.11 109.22) (width 0.2) (layer "F.Cu") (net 21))
 (segment (start 114.3 78.74) (end 118.11 78.74) (width 0.2) (layer "F.Cu") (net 9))
 (segment (start 114.3 83.82) (end 118.11 83.82) (width 0.2) (layer "F.Cu") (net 11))
 (segment (start 114.3 121.92) (end 118.11 121.92) (width 0.2) (layer "F.Cu") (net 26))
 (segment (start 114.3 91.44) (end 118.11 91.44) (width 0.2) (layer "F.Cu") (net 14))
 (segment (start 114.3 88.9) (end 118.11 88.9) (width 0.2) (layer "F.Cu") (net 13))
 (segment (start 114.3 93.98) (end 118.11 93.98) (width 0.2) (layer "F.Cu") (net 15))
 (segment (start 114.3 96.52) (end 118.11 96.52) (width 0.2) (layer "F.Cu") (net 16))
 (segment (start 114.3 116.84) (end 118.11 116.84) (width 0.2) (layer "F.Cu") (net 24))
 (segment (start 114.3 76.2) (end 118.11 76.2) (width 0.2) (layer "F.Cu") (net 8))
 (segment (start 128.27 91.44) (end 132.08 91.44) (width 0.2) (layer "F.Cu") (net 33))
 (segment (start 128.27 99.06) (end 127.119 100.211) (width 0.2) (layer "F.Cu") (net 36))
 (segment (start 123.19 101.87724) (end 123.19 112.9025) (width 0.2) (layer "F.Cu") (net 36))
 (segment (start 127.119 100.211) (end 124.85624 100.211) (width 0.2) (layer "F.Cu") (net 36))
 (segment (start 123.19 112.9025) (end 121.19 114.9025) (width 0.2) (layer "F.Cu") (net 36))
 (segment (start 128.27 99.06) (end 132.08 99.06) (width 0.2) (layer "F.Cu") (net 36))
 (segment (start 124.85624 100.211) (end 123.19 101.87724) (width 0.2) (layer "F.Cu") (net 36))
 (segment (start 123.825 79.375) (end 128.27 83.82) (width 0.2) (layer "F.Cu") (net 5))
 (segment (start 128.27 83.82) (end 132.08 83.82) (width 0.2) (layer "F.Cu") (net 5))
 (segment (start 128.27 81.28) (end 132.08 81.28) (width 0.2) (layer "F.Cu") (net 30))
 (segment (start 128.27 109.22) (end 132.08 109.22) (width 0.2) (layer "F.Cu") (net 40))
 (segment (start 126.365 113.7275) (end 125.19 114.9025) (width 0.2) (layer "F.Cu") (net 38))
 (segment (start 128.27 104.14) (end 126.365 106.045) (width 0.2) (layer "F.Cu") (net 38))
 (segment (start 126.365 106.045) (end 126.365 113.7275) (width 0.2) (layer "F.Cu") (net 38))
 (segment (start 128.27 104.14) (end 132.08 104.14) (width 0.2) (layer "F.Cu") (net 38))
 (segment (start 128.27 76.2) (end 132.08 76.2) (width 0.2) (layer "F.Cu") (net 28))
 (segment (start 128.27 73.66) (end 132.08 73.66) (width 0.2) (layer "F.Cu") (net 27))
 (segment (start 128.27 86.36) (end 132.08 86.36) (width 0.2) (layer "F.Cu") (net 31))
 (segment (start 128.27 119.38) (end 132.08 119.38) (width 0.2) (layer "F.Cu") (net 44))
 (segment (start 128.27 101.6) (end 132.08 101.6) (width 0.2) (layer "F.Cu") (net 37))
 (segment (start 128.27 88.9) (end 132.08 88.9) (width 0.2) (layer "F.Cu") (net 32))
 (segment (start 128.27 121.92) (end 132.08 121.92) (width 0.2) (layer "F.Cu") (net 45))
 (segment (start 128.27 93.98) (end 132.08 93.98) (width 0.2) (layer "F.Cu") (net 34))
 (segment (start 128.27 116.84) (end 132.08 116.84) (width 0.2) (layer "F.Cu") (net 43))
 (segment (start 128.27 114.3) (end 132.08 114.3) (width 0.2) (layer "F.Cu") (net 42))
 (segment (start 128.27 96.52) (end 132.08 96.52) (width 0.2) (layer "F.Cu") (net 35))
 (segment (start 128.27 111.76) (end 132.08 111.76) (width 0.2) (layer "F.Cu") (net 41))
 (segment (start 128.27 106.68) (end 132.08 106.68) (width 0.2) (layer "F.Cu") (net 39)))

